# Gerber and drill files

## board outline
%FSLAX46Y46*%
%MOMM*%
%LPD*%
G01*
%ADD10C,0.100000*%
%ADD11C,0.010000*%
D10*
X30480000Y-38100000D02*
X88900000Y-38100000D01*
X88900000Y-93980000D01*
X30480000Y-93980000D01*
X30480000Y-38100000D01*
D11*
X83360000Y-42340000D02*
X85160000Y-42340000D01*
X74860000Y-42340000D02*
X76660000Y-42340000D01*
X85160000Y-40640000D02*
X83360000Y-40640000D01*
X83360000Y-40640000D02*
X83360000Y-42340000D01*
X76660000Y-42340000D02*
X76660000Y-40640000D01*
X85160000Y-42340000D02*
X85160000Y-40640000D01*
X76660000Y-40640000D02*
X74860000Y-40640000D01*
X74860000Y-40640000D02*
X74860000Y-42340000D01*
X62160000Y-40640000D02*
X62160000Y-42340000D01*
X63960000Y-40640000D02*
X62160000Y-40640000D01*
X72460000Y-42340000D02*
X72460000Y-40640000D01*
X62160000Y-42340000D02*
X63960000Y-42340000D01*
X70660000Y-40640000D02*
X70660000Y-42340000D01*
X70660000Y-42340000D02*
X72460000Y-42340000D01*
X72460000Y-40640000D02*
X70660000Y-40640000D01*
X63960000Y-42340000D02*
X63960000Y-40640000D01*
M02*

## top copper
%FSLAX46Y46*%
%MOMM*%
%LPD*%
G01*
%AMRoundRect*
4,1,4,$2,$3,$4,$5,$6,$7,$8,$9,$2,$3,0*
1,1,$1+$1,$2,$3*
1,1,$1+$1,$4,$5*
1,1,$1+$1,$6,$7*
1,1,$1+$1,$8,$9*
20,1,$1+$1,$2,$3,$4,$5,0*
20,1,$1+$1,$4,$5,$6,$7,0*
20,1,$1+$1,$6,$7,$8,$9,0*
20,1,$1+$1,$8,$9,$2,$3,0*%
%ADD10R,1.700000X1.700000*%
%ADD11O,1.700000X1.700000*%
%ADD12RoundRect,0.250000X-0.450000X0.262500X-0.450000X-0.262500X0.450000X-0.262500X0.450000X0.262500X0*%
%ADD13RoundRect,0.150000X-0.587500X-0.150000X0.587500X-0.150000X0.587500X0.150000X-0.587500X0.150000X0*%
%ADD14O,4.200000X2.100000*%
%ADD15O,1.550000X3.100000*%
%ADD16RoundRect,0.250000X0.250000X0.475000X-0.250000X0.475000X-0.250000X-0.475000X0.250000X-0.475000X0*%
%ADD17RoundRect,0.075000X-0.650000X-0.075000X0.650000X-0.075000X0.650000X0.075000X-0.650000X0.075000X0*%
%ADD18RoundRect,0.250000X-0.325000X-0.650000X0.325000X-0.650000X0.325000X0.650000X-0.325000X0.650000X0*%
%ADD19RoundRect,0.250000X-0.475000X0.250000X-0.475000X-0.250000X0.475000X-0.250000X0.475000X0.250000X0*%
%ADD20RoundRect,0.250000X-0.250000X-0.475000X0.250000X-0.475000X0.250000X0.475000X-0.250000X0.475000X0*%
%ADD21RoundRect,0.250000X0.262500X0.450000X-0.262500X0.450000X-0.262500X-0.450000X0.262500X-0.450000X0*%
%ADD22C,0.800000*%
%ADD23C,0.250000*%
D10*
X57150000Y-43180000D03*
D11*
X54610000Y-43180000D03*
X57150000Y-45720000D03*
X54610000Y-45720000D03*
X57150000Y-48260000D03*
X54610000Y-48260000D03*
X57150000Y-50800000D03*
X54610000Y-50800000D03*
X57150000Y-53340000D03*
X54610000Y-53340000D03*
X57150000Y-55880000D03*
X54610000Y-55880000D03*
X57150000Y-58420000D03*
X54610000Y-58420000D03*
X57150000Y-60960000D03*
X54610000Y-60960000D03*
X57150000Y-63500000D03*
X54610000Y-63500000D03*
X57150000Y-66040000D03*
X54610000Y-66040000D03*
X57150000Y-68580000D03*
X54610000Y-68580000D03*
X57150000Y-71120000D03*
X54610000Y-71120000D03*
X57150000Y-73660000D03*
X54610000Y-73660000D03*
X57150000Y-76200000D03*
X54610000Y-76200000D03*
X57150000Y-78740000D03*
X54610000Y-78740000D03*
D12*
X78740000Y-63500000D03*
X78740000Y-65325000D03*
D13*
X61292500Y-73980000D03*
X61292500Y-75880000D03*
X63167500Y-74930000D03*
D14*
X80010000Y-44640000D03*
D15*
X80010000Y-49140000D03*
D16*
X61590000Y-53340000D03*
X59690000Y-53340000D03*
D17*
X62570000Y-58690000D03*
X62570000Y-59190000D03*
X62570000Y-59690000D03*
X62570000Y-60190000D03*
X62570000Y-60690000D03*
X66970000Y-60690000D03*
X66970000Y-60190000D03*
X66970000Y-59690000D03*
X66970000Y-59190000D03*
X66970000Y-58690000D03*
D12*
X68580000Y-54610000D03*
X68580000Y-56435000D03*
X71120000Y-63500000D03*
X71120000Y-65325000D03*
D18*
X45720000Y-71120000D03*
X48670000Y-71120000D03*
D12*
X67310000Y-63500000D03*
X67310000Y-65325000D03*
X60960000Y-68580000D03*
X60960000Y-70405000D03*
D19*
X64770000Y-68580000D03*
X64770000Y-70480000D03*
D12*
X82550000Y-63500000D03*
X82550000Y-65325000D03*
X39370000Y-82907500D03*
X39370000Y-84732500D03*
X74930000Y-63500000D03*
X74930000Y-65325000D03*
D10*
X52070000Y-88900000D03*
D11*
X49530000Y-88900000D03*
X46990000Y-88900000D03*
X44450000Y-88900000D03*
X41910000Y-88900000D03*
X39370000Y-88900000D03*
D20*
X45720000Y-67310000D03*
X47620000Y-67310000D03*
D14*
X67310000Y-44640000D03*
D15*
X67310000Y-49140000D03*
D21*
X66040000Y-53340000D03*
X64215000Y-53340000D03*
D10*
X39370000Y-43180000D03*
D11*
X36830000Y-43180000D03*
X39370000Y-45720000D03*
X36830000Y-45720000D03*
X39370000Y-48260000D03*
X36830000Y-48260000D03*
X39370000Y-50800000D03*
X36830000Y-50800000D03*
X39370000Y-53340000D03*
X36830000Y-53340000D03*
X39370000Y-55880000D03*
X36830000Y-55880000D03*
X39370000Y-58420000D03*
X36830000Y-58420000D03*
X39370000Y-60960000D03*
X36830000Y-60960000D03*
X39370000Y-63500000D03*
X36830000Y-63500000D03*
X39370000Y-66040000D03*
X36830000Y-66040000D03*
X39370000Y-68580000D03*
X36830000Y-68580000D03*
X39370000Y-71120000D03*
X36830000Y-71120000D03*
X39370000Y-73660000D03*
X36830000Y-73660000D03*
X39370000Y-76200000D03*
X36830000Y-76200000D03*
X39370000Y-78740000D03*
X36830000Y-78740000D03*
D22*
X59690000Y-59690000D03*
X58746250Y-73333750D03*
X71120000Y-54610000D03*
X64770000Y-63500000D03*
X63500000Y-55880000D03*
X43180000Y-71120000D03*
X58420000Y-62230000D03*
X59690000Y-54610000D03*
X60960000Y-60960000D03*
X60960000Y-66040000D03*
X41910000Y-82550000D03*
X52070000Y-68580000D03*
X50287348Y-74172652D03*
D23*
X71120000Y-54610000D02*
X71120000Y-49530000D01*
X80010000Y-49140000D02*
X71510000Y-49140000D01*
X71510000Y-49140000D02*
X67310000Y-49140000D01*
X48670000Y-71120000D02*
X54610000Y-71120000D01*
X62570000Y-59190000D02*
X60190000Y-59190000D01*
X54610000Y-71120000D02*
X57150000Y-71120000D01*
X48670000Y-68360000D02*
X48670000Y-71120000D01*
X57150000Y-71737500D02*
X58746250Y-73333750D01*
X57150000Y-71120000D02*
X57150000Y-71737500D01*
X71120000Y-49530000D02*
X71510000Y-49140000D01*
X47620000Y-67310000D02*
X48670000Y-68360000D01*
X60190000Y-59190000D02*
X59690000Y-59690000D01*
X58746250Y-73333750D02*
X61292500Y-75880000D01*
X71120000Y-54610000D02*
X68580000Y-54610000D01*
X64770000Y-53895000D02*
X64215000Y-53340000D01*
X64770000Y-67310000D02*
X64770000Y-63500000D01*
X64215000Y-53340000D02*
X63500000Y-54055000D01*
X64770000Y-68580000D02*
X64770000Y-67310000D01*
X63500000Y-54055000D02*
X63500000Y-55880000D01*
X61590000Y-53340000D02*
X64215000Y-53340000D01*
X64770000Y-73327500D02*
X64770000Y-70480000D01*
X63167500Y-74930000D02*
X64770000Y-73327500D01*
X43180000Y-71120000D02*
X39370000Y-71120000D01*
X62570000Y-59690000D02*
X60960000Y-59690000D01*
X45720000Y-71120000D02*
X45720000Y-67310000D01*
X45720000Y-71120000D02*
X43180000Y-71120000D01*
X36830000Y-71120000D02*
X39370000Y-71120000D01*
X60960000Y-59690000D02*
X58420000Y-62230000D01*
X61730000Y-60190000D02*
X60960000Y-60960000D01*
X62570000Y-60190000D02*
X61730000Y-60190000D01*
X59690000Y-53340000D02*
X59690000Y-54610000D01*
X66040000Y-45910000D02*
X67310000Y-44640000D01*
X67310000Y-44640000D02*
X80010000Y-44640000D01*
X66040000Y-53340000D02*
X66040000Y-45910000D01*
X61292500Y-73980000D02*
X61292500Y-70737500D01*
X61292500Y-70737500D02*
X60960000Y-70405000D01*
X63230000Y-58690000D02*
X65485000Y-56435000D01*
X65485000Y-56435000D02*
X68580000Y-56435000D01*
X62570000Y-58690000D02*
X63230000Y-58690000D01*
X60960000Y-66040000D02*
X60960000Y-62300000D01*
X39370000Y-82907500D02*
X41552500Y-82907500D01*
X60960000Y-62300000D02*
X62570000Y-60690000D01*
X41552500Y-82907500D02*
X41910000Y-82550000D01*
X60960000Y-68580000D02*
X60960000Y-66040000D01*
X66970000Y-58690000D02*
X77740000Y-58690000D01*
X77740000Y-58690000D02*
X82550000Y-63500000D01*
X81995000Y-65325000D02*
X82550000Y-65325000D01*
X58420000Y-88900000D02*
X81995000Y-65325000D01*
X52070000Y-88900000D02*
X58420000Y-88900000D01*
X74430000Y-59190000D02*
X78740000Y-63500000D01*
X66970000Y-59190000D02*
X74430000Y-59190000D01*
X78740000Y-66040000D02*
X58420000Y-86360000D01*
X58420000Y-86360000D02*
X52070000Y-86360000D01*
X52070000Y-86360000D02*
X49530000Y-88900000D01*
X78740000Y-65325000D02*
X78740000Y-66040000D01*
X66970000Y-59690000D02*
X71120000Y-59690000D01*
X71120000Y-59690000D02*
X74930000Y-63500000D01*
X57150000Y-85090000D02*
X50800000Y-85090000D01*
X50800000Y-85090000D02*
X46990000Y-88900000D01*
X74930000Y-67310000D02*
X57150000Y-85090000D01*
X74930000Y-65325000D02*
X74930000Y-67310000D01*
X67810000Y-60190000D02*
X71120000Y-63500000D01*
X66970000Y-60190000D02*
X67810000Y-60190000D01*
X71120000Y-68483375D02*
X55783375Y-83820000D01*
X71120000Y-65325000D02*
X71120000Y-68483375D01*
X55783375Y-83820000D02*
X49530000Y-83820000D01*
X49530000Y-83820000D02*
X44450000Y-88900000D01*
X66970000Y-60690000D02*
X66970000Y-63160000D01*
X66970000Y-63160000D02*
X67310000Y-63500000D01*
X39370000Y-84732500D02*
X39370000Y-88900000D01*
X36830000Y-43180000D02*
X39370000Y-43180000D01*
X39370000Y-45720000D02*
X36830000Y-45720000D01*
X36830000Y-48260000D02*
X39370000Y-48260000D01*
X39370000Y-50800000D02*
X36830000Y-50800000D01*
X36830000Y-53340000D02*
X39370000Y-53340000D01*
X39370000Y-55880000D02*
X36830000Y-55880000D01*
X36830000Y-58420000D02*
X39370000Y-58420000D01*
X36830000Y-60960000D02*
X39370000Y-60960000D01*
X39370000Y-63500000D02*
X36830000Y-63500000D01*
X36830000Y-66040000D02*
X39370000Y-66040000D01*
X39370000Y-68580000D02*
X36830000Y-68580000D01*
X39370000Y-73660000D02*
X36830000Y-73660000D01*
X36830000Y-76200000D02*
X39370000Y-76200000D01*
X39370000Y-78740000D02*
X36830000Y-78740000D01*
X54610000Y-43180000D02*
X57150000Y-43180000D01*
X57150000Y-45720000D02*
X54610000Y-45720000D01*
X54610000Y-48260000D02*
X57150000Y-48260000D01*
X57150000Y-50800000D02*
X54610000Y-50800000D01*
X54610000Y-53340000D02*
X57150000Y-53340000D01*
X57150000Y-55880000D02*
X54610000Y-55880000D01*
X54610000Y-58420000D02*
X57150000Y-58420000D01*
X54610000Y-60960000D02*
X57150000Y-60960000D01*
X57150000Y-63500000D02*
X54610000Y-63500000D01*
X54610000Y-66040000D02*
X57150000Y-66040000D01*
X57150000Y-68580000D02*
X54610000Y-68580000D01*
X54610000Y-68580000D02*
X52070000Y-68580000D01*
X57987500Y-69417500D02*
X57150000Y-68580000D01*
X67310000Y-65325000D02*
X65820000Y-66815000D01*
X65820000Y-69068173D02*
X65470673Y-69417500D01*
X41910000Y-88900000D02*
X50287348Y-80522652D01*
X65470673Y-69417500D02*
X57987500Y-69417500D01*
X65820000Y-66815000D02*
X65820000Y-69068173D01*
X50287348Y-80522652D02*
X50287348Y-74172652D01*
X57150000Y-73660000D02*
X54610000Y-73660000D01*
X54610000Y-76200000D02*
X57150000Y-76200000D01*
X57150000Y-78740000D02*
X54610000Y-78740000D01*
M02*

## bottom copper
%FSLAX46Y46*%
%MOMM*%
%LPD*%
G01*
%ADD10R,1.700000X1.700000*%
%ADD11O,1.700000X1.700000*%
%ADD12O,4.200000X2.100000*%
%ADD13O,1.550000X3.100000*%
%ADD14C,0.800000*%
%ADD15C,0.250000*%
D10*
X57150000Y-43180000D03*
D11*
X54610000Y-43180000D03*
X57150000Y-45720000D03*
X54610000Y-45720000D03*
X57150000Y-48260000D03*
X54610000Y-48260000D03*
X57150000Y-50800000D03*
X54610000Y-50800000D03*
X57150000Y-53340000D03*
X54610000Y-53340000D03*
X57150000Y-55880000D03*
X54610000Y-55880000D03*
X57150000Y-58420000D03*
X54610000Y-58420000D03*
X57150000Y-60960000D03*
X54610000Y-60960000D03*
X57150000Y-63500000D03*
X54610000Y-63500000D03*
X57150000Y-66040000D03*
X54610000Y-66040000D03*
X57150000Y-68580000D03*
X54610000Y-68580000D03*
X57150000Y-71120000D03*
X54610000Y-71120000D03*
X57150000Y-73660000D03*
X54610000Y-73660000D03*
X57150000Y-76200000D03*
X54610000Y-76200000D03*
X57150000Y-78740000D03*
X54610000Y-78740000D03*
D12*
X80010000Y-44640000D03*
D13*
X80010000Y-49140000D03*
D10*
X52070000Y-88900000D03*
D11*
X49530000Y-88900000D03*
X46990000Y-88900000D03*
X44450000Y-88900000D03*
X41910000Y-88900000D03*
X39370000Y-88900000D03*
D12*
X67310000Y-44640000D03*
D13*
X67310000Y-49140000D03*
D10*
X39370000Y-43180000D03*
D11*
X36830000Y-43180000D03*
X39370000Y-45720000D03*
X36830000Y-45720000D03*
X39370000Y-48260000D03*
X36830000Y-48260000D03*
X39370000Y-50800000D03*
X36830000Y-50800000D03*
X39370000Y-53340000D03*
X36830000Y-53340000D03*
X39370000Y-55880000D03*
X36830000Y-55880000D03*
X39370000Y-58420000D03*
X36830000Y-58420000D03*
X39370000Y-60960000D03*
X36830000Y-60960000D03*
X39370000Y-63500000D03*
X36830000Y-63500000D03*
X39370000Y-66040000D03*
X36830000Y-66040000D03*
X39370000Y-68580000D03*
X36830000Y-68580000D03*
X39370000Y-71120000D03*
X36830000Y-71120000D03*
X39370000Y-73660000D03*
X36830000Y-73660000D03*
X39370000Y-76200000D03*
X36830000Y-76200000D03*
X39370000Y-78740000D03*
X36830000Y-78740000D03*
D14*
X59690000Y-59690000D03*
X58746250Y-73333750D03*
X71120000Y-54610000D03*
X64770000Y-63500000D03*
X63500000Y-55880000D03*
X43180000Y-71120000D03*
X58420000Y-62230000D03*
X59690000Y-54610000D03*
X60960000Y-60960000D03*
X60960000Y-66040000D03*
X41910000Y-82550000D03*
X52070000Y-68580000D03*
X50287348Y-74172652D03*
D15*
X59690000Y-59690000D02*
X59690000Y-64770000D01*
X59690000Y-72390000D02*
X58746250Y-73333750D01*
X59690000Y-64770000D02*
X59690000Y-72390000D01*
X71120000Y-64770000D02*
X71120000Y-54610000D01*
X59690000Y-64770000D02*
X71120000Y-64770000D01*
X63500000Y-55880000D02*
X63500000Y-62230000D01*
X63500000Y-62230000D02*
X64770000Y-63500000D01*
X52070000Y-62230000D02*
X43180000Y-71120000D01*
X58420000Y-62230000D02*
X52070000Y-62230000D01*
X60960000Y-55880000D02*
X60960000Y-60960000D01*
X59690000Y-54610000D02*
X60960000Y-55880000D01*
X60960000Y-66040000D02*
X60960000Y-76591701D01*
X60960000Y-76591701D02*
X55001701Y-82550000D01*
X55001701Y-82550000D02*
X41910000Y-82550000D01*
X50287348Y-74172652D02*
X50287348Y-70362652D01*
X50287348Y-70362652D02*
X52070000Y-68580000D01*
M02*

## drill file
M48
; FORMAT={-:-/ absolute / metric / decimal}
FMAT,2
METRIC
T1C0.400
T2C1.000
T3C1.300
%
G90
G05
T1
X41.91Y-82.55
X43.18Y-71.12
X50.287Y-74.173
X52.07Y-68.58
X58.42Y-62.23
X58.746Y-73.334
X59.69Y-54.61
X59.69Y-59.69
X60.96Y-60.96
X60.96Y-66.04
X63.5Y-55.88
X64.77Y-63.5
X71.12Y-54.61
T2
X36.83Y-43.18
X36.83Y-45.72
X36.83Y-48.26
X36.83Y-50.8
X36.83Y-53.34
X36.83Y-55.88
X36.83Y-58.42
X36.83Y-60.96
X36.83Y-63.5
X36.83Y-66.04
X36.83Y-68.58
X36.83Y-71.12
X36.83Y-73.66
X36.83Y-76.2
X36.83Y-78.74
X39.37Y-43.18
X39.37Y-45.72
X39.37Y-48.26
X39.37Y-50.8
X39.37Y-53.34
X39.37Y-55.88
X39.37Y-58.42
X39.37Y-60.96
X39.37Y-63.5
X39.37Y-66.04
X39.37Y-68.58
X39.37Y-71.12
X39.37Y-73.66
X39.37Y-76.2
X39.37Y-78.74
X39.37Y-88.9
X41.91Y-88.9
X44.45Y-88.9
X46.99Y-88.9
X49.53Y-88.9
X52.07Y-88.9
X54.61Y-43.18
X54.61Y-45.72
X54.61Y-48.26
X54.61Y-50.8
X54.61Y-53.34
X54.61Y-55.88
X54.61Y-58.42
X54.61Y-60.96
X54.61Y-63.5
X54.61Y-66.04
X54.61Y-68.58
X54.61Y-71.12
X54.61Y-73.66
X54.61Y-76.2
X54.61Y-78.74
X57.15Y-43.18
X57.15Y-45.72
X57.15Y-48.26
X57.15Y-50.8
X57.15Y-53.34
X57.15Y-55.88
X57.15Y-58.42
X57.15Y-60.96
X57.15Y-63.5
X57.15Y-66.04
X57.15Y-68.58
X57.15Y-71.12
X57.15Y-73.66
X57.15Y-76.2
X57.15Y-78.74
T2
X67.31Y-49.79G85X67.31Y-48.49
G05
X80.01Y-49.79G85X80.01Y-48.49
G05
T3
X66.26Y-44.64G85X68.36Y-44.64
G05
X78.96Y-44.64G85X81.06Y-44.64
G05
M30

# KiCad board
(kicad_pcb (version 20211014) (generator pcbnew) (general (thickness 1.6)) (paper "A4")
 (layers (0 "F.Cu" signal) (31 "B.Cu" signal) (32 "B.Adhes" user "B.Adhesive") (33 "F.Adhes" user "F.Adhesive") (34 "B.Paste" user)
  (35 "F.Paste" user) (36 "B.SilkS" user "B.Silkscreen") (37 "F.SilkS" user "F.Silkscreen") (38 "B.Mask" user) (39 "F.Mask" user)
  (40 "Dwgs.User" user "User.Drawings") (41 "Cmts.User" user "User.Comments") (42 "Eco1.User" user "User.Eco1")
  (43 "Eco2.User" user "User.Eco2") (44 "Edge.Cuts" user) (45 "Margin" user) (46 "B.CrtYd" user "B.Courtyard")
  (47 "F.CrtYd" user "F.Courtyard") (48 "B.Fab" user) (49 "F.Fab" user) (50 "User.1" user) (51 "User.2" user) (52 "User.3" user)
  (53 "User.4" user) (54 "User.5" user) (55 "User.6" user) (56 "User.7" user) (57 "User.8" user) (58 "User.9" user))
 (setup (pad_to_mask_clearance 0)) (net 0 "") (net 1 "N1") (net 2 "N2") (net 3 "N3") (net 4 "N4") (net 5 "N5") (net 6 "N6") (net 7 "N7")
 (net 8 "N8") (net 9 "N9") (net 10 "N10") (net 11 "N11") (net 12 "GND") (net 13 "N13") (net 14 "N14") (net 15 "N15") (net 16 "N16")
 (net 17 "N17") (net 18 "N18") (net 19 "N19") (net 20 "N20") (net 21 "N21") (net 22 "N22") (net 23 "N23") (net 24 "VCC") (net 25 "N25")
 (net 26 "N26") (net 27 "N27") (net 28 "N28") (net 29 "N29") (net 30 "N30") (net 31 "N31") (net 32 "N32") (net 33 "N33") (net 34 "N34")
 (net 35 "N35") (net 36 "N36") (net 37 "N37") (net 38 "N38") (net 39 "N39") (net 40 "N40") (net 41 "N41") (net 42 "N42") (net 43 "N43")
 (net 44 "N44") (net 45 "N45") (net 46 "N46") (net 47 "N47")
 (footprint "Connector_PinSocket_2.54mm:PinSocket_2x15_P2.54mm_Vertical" (layer "F.Cu") (at 57.15 43.18)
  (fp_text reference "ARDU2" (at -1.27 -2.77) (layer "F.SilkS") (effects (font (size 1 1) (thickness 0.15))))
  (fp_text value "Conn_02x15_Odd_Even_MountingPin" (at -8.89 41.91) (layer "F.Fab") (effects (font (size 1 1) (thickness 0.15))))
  (pad "1" thru_hole rect (at 0 0) (size 1.7 1.7) (drill 1) (layers *.Cu *.Mask) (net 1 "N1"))
  (pad "2" thru_hole oval (at -2.54 0) (size 1.7 1.7) (drill 1) (layers *.Cu *.Mask) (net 1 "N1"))
  (pad "3" thru_hole oval (at 0 2.54) (size 1.7 1.7) (drill 1) (layers *.Cu *.Mask) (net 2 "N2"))
  (pad "4" thru_hole oval (at -2.54 2.54) (size 1.7 1.7) (drill 1) (layers *.Cu *.Mask) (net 2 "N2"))
  (pad "5" thru_hole oval (at 0 5.08) (size 1.7 1.7) (drill 1) (layers *.Cu *.Mask) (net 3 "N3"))
  (pad "6" thru_hole oval (at -2.54 5.08) (size 1.7 1.7) (drill 1) (layers *.Cu *.Mask) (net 3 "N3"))
  (pad "7" thru_hole oval (at 0 7.62) (size 1.7 1.7) (drill 1) (layers *.Cu *.Mask) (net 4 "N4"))
  (pad "8" thru_hole oval (at -2.54 7.62) (size 1.7 1.7) (drill 1) (layers *.Cu *.Mask) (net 4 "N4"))
  (pad "9" thru_hole oval (at 0 10.16) (size 1.7 1.7) (drill 1) (layers *.Cu *.Mask) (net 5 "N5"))
  (pad "10" thru_hole oval (at -2.54 10.16) (size 1.7 1.7) (drill 1) (layers *.Cu *.Mask) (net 5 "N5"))
  (pad "11" thru_hole oval (at 0 12.7) (size 1.7 1.7) (drill 1) (layers *.Cu *.Mask) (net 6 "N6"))
  (pad "12" thru_hole oval (at -2.54 12.7) (size 1.7 1.7) (drill 1) (layers *.Cu *.Mask) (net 6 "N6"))
  (pad "13" thru_hole oval (at 0 15.24) (size 1.7 1.7) (drill 1) (layers *.Cu *.Mask) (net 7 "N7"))
  (pad "14" thru_hole oval (at -2.54 15.24) (size 1.7 1.7) (drill 1) (layers *.Cu *.Mask) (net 7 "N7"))
  (pad "15" thru_hole oval (at 0 17.78) (size 1.7 1.7) (drill 1) (layers *.Cu *.Mask) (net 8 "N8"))
  (pad "16" thru_hole oval (at -2.54 17.78) (size 1.7 1.7) (drill 1) (layers *.Cu *.Mask) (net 8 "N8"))
  (pad "17" thru_hole oval (at 0 20.32) (size 1.7 1.7) (drill 1) (layers *.Cu *.Mask) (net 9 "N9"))
  (pad "18" thru_hole oval (at -2.54 20.32) (size 1.7 1.7) (drill 1) (layers *.Cu *.Mask) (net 9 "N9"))
  (pad "19" thru_hole oval (at 0 22.86) (size 1.7 1.7) (drill 1) (layers *.Cu *.Mask) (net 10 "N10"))
  (pad "20" thru_hole oval (at -2.54 22.86) (size 1.7 1.7) (drill 1) (layers *.Cu *.Mask) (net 10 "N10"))
  (pad "21" thru_hole oval (at 0 25.4) (size 1.7 1.7) (drill 1) (layers *.Cu *.Mask) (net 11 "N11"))
  (pad "22" thru_hole oval (at -2.54 25.4) (size 1.7 1.7) (drill 1) (layers *.Cu *.Mask) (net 11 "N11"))
  (pad "23" thru_hole oval (at 0 27.94) (size 1.7 1.7) (drill 1) (layers *.Cu *.Mask) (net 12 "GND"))
  (pad "24" thru_hole oval (at -2.54 27.94) (size 1.7 1.7) (drill 1) (layers *.Cu *.Mask) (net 12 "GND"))
  (pad "25" thru_hole oval (at 0 30.48) (size 1.7 1.7) (drill 1) (layers *.Cu *.Mask) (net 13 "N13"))
  (pad "26" thru_hole oval (at -2.54 30.48) (size 1.7 1.7) (drill 1) (layers *.Cu *.Mask) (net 13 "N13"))
  (pad "27" thru_hole oval (at 0 33.02) (size 1.7 1.7) (drill 1) (layers *.Cu *.Mask) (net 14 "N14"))
  (pad "28" thru_hole oval (at -2.54 33.02) (size 1.7 1.7) (drill 1) (layers *.Cu *.Mask) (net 14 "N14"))
  (pad "29" thru_hole oval (at 0 35.56) (size 1.7 1.7) (drill 1) (layers *.Cu *.Mask) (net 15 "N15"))
  (pad "30" thru_hole oval (at -2.54 35.56) (size 1.7 1.7) (drill 1) (layers *.Cu *.Mask) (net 15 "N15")))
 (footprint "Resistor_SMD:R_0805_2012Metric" (layer "F.Cu") (at 78.74 64.4125 -90)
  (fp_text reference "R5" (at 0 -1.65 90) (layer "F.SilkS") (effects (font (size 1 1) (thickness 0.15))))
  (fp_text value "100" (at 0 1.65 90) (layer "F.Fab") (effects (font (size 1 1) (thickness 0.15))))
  (pad "1" smd roundrect (at -0.9125 0 270) (size 1.025 1.4) (layers "F.Cu" "F.Paste" "F.Mask") (roundrect_rratio 0.243902) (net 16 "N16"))
  (pad "2" smd roundrect (at 0.9125 0 270) (size 1.025 1.4) (layers "F.Cu" "F.Paste" "F.Mask") (roundrect_rratio 0.243902) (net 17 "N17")))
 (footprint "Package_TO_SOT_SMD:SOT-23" (layer "F.Cu") (at 62.23 74.93)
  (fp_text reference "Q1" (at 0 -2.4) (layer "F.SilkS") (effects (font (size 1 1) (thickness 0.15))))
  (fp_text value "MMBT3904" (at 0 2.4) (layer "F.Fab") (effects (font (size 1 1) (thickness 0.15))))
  (pad "1" smd roundrect (at -0.9375 -0.95) (size 1.475 0.6) (layers "F.Cu" "F.Paste" "F.Mask") (roundrect_rratio 0.25) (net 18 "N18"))
  (pad "2" smd roundrect (at -0.9375 0.95) (size 1.475 0.6) (layers "F.Cu" "F.Paste" "F.Mask") (roundrect_rratio 0.25) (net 12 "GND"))
  (pad "3" smd roundrect (at 0.9375 0) (size 1.475 0.6) (layers "F.Cu" "F.Paste" "F.Mask") (roundrect_rratio 0.25) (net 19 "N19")))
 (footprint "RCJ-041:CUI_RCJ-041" (layer "F.Cu") (at 80.01 40.64 90)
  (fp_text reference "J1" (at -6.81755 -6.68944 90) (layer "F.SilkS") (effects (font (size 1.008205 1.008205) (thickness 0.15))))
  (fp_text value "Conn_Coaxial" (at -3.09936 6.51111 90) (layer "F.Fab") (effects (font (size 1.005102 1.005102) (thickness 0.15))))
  (fp_line (start -1.7 3.35) (end -1.7 5.15) (layer "Edge.Cuts") (width 0.01))
  (fp_line (start -1.7 -5.15) (end -1.7 -3.35) (layer "Edge.Cuts") (width 0.01))
  (fp_line (start 0 5.15) (end 0 3.35) (layer "Edge.Cuts") (width 0.01))
  (fp_line (start 0 3.35) (end -1.7 3.35) (layer "Edge.Cuts") (width 0.01))
  (fp_line (start -1.7 -3.35) (end 0 -3.35) (layer "Edge.Cuts") (width 0.01))
  (fp_line (start -1.7 5.15) (end 0 5.15) (layer "Edge.Cuts") (width 0.01))
  (fp_line (start 0 -3.35) (end 0 -5.15) (layer "Edge.Cuts") (width 0.01))
  (fp_line (start 0 -5.15) (end -1.7 -5.15) (layer "Edge.Cuts") (width 0.01))
  (pad "1" thru_hole oval locked (at -4 0 90) (size 2.1 4.2) (drill oval 1.3 3.4) (layers *.Cu *.Mask) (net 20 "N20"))
  (pad "2" thru_hole oval locked (at -8.5 0 90) (size 3.1 1.55) (drill oval 2.3 1) (layers *.Cu *.Mask) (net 12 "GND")))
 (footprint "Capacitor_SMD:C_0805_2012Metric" (layer "F.Cu") (at 60.64 53.34 180)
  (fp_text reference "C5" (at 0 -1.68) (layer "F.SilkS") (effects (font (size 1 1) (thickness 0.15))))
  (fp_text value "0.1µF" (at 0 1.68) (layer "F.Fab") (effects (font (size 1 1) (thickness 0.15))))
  (pad "1" smd roundrect (at -0.95 0 180) (size 1 1.45) (layers "F.Cu" "F.Paste" "F.Mask") (roundrect_rratio 0.25) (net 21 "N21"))
  (pad "2" smd roundrect (at 0.95 0 180) (size 1 1.45) (layers "F.Cu" "F.Paste" "F.Mask") (roundrect_rratio 0.25) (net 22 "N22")))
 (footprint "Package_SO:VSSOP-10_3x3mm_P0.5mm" (layer "F.Cu") (at 64.77 59.69)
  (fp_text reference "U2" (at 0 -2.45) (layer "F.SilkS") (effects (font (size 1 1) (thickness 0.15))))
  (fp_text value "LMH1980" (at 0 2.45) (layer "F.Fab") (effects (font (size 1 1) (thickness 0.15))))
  (pad "1" smd roundrect (at -2.2 -1) (size 1.45 0.3) (layers "F.Cu" "F.Paste" "F.Mask") (roundrect_rratio 0.25) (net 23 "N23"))
  (pad "2" smd roundrect (at -2.2 -0.5) (size 1.45 0.3) (layers "F.Cu" "F.Paste" "F.Mask") (roundrect_rratio 0.25) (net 12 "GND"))
  (pad "3" smd roundrect (at -2.2 0) (size 1.45 0.3) (layers "F.Cu" "F.Paste" "F.Mask") (roundrect_rratio 0.25) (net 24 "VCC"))
  (pad "4" smd roundrect (at -2.2 0.5) (size 1.45 0.3) (layers "F.Cu" "F.Paste" "F.Mask") (roundrect_rratio 0.25) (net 22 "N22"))
  (pad "5" smd roundrect (at -2.2 1) (size 1.45 0.3) (layers "F.Cu" "F.Paste" "F.Mask") (roundrect_rratio 0.25) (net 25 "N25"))
  (pad "6" smd roundrect (at 2.2 1) (size 1.45 0.3) (layers "F.Cu" "F.Paste" "F.Mask") (roundrect_rratio 0.25) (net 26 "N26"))
  (pad "7" smd roundrect (at 2.2 0.5) (size 1.45 0.3) (layers "F.Cu" "F.Paste" "F.Mask") (roundrect_rratio 0.25) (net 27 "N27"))
  (pad "8" smd roundrect (at 2.2 0) (size 1.45 0.3) (layers "F.Cu" "F.Paste" "F.Mask") (roundrect_rratio 0.25) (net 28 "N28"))
  (pad "9" smd roundrect (at 2.2 -0.5) (size 1.45 0.3) (layers "F.Cu" "F.Paste" "F.Mask") (roundrect_rratio 0.25) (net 16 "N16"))
  (pad "10" smd roundrect (at 2.2 -1) (size 1.45 0.3) (layers "F.Cu" "F.Paste" "F.Mask") (roundrect_rratio 0.25) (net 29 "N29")))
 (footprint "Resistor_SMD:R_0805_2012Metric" (layer "F.Cu") (at 68.58 55.5225 -90)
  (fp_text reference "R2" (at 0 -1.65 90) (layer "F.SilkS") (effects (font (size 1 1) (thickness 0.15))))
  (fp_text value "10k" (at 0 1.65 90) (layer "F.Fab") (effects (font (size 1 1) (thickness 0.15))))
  (pad "1" smd roundrect (at -0.9125 0 270) (size 1.025 1.4) (layers "F.Cu" "F.Paste" "F.Mask") (roundrect_rratio 0.243902) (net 12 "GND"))
  (pad "2" smd roundrect (at 0.9125 0 270) (size 1.025 1.4) (layers "F.Cu" "F.Paste" "F.Mask") (roundrect_rratio 0.243902) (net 23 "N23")))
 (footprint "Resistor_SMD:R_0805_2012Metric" (layer "F.Cu") (at 71.12 64.4125 -90)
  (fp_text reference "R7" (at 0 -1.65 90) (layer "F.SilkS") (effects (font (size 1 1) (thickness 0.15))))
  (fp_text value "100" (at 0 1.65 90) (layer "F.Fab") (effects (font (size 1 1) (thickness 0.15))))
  (pad "1" smd roundrect (at -0.9125 0 270) (size 1.025 1.4) (layers "F.Cu" "F.Paste" "F.Mask") (roundrect_rratio 0.243902) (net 27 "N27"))
  (pad "2" smd roundrect (at 0.9125 0 270) (size 1.025 1.4) (layers "F.Cu" "F.Paste" "F.Mask") (roundrect_rratio 0.243902) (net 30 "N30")))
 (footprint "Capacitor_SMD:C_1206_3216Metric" (layer "F.Cu") (at 47.195 71.12)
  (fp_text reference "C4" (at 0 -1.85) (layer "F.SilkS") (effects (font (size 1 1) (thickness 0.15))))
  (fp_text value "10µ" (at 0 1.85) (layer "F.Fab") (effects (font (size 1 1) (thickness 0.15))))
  (pad "1" smd roundrect (at -1.475 0) (size 1.15 1.8) (layers "F.Cu" "F.Paste" "F.Mask") (roundrect_rratio 0.217391) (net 24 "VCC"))
  (pad "2" smd roundrect (at 1.475 0) (size 1.15 1.8) (layers "F.Cu" "F.Paste" "F.Mask") (roundrect_rratio 0.217391) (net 12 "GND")))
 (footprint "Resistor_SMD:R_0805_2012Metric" (layer "F.Cu") (at 67.31 64.4125 -90)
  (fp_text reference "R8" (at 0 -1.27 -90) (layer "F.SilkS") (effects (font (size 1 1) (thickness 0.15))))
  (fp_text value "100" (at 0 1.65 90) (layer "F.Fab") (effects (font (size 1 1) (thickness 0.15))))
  (pad "1" smd roundrect (at -0.9125 0 270) (size 1.025 1.4) (layers "F.Cu" "F.Paste" "F.Mask") (roundrect_rratio 0.243902) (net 26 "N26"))
  (pad "2" smd roundrect (at 0.9125 0 270) (size 1.025 1.4) (layers "F.Cu" "F.Paste" "F.Mask") (roundrect_rratio 0.243902) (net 11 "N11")))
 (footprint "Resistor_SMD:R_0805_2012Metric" (layer "F.Cu") (at 60.96 69.4925 -90)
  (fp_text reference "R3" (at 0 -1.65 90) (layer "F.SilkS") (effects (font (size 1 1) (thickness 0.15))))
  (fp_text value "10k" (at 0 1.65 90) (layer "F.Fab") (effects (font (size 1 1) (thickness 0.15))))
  (pad "1" smd roundrect (at -0.9125 0 270) (size 1.025 1.4) (layers "F.Cu" "F.Paste" "F.Mask") (roundrect_rratio 0.243902) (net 25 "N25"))
  (pad "2" smd roundrect (at 0.9125 0 270) (size 1.025 1.4) (layers "F.Cu" "F.Paste" "F.Mask") (roundrect_rratio 0.243902) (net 18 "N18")))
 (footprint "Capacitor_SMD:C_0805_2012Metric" (layer "F.Cu") (at 64.77 69.53 -90)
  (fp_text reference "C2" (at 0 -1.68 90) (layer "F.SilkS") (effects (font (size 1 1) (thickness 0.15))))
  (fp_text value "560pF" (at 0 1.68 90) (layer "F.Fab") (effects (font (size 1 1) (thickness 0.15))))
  (pad "1" smd roundrect (at -0.95 0 270) (size 1 1.45) (layers "F.Cu" "F.Paste" "F.Mask") (roundrect_rratio 0.25) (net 21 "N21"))
  (pad "2" smd roundrect (at 0.95 0 270) (size 1 1.45) (layers "F.Cu" "F.Paste" "F.Mask") (roundrect_rratio 0.25) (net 19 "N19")))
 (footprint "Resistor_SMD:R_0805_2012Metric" (layer "F.Cu") (at 82.55 64.4125 -90)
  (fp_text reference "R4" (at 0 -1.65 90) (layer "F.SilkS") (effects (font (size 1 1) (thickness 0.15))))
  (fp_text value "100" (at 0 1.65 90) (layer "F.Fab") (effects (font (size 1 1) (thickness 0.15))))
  (pad "1" smd roundrect (at -0.9125 0 270) (size 1.025 1.4) (layers "F.Cu" "F.Paste" "F.Mask") (roundrect_rratio 0.243902) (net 29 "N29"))
  (pad "2" smd roundrect (at 0.9125 0 270) (size 1.025 1.4) (layers "F.Cu" "F.Paste" "F.Mask") (roundrect_rratio 0.243902) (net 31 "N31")))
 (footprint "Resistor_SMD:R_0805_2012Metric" (layer "F.Cu") (at 39.37 83.82 -90)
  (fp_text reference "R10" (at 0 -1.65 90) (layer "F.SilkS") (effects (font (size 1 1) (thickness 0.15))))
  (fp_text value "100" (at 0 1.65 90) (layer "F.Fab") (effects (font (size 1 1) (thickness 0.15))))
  (pad "1" smd roundrect (at -0.9125 0 270) (size 1.025 1.4) (layers "F.Cu" "F.Paste" "F.Mask") (roundrect_rratio 0.243902) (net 25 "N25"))
  (pad "2" smd roundrect (at 0.9125 0 270) (size 1.025 1.4) (layers "F.Cu" "F.Paste" "F.Mask") (roundrect_rratio 0.243902) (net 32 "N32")))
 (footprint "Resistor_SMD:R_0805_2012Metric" (layer "F.Cu") (at 74.93 64.4125 -90)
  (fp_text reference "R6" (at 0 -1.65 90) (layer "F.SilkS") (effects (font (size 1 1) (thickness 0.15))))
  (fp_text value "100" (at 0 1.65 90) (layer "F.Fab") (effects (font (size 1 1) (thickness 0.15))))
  (pad "1" smd roundrect (at -0.9125 0 270) (size 1.025 1.4) (layers "F.Cu" "F.Paste" "F.Mask") (roundrect_rratio 0.243902) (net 28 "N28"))
  (pad "2" smd roundrect (at 0.9125 0 270) (size 1.025 1.4) (layers "F.Cu" "F.Paste" "F.Mask") (roundrect_rratio 0.243902) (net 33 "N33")))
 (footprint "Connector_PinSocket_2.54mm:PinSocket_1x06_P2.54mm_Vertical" (layer "F.Cu") (at 52.07 88.9 -90)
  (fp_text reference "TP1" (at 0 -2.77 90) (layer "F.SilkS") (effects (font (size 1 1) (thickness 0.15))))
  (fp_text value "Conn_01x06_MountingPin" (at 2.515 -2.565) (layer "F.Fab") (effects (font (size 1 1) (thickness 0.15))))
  (pad "1" thru_hole rect (at 0 0 270) (size 1.7 1.7) (drill 1) (layers *.Cu *.Mask) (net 31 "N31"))
  (pad "2" thru_hole oval (at 0 2.54 270) (size 1.7 1.7) (drill 1) (layers *.Cu *.Mask) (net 17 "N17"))
  (pad "3" thru_hole oval (at 0 5.08 270) (size 1.7 1.7) (drill 1) (layers *.Cu *.Mask) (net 33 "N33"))
  (pad "4" thru_hole oval (at 0 7.62 270) (size 1.7 1.7) (drill 1) (layers *.Cu *.Mask) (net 30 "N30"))
  (pad "5" thru_hole oval (at 0 10.16 270) (size 1.7 1.7) (drill 1) (layers *.Cu *.Mask) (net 11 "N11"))
  (pad "6" thru_hole oval (at 0 12.7 270) (size 1.7 1.7) (drill 1) (layers *.Cu *.Mask) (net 32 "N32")))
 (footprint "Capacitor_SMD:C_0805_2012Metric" (layer "F.Cu") (at 46.67 67.31)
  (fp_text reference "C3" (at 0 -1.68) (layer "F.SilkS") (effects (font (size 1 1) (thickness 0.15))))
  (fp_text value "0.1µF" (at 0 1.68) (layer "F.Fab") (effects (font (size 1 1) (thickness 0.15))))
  (pad "1" smd roundrect (at -0.95 0) (size 1 1.45) (layers "F.Cu" "F.Paste" "F.Mask") (roundrect_rratio 0.25) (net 24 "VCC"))
  (pad "2" smd roundrect (at 0.95 0) (size 1 1.45) (layers "F.Cu" "F.Paste" "F.Mask") (roundrect_rratio 0.25) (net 12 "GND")))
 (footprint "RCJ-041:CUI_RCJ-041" (layer "F.Cu") (at 67.31 40.64 90)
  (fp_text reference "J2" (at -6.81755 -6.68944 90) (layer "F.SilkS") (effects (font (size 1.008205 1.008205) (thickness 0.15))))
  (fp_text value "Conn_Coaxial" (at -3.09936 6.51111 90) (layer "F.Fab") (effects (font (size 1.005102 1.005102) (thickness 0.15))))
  (fp_line (start 0 -5.15) (end -1.7 -5.15) (layer "Edge.Cuts") (width 0.01))
  (fp_line (start 0 -3.35) (end 0 -5.15) (layer "Edge.Cuts") (width 0.01))
  (fp_line (start -1.7 5.15) (end 0 5.15) (layer "Edge.Cuts") (width 0.01))
  (fp_line (start -1.7 -5.15) (end -1.7 -3.35) (layer "Edge.Cuts") (width 0.01))
  (fp_line (start 0 3.35) (end -1.7 3.35) (layer "Edge.Cuts") (width 0.01))
  (fp_line (start -1.7 3.35) (end -1.7 5.15) (layer "Edge.Cuts") (width 0.01))
  (fp_line (start 0 5.15) (end 0 3.35) (layer "Edge.Cuts") (width 0.01))
  (fp_line (start -1.7 -3.35) (end 0 -3.35) (layer "Edge.Cuts") (width 0.01))
  (pad "1" thru_hole oval locked (at -4 0 90) (size 2.1 4.2) (drill oval 1.3 3.4) (layers *.Cu *.Mask) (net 20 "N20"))
  (pad "2" thru_hole oval locked (at -8.5 0 90) (size 3.1 1.55) (drill oval 2.3 1) (layers *.Cu *.Mask) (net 12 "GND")))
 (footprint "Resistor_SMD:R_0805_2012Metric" (layer "F.Cu") (at 65.1275 53.34 180)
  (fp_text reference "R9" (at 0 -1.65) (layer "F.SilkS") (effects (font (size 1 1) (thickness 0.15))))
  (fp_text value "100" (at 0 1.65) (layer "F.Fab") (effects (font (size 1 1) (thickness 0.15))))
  (pad "1" smd roundrect (at -0.9125 0 180) (size 1.025 1.4) (layers "F.Cu" "F.Paste" "F.Mask") (roundrect_rratio 0.243902) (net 20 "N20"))
  (pad "2" smd roundrect (at 0.9125 0 180) (size 1.025 1.4) (layers "F.Cu" "F.Paste" "F.Mask") (roundrect_rratio 0.243902) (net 21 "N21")))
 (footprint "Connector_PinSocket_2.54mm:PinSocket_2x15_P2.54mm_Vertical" (layer "F.Cu") (at 39.37 43.18)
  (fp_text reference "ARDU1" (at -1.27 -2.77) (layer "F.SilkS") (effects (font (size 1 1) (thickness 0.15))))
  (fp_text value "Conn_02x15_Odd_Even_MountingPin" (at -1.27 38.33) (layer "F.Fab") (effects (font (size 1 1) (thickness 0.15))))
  (pad "1" thru_hole rect (at 0 0) (size 1.7 1.7) (drill 1) (layers *.Cu *.Mask) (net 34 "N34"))
  (pad "2" thru_hole oval (at -2.54 0) (size 1.7 1.7) (drill 1) (layers *.Cu *.Mask) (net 34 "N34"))
  (pad "3" thru_hole oval (at 0 2.54) (size 1.7 1.7) (drill 1) (layers *.Cu *.Mask) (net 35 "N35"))
  (pad "4" thru_hole oval (at -2.54 2.54) (size 1.7 1.7) (drill 1) (layers *.Cu *.Mask) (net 35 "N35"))
  (pad "5" thru_hole oval (at 0 5.08) (size 1.7 1.7) (drill 1) (layers *.Cu *.Mask) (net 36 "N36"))
  (pad "6" thru_hole oval (at -2.54 5.08) (size 1.7 1.7) (drill 1) (layers *.Cu *.Mask) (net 36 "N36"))
  (pad "7" thru_hole oval (at 0 7.62) (size 1.7 1.7) (drill 1) (layers *.Cu *.Mask) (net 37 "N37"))
  (pad "8" thru_hole oval (at -2.54 7.62) (size 1.7 1.7) (drill 1) (layers *.Cu *.Mask) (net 37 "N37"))
  (pad "9" thru_hole oval (at 0 10.16) (size 1.7 1.7) (drill 1) (layers *.Cu *.Mask) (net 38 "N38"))
  (pad "10" thru_hole oval (at -2.54 10.16) (size 1.7 1.7) (drill 1) (layers *.Cu *.Mask) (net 38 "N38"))
  (pad "11" thru_hole oval (at 0 12.7) (size 1.7 1.7) (drill 1) (layers *.Cu *.Mask) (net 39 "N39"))
  (pad "12" thru_hole oval (at -2.54 12.7) (size 1.7 1.7) (drill 1) (layers *.Cu *.Mask) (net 39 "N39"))
  (pad "13" thru_hole oval (at 0 15.24) (size 1.7 1.7) (drill 1) (layers *.Cu *.Mask) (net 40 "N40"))
  (pad "14" thru_hole oval (at -2.54 15.24) (size 1.7 1.7) (drill 1) (layers *.Cu *.Mask) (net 40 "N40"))
  (pad "15" thru_hole oval (at 0 17.78) (size 1.7 1.7) (drill 1) (layers *.Cu *.Mask) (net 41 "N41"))
  (pad "16" thru_hole oval (at -2.54 17.78) (size 1.7 1.7) (drill 1) (layers *.Cu *.Mask) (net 41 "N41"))
  (pad "17" thru_hole oval (at 0 20.32) (size 1.7 1.7) (drill 1) (layers *.Cu *.Mask) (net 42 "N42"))
  (pad "18" thru_hole oval (at -2.54 20.32) (size 1.7 1.7) (drill 1) (layers *.Cu *.Mask) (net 42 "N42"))
  (pad "19" thru_hole oval (at 0 22.86) (size 1.7 1.7) (drill 1) (layers *.Cu *.Mask) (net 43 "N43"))
  (pad "20" thru_hole oval (at -2.54 22.86) (size 1.7 1.7) (drill 1) (layers *.Cu *.Mask) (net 43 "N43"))
  (pad "21" thru_hole oval (at 0 25.4) (size 1.7 1.7) (drill 1) (layers *.Cu *.Mask) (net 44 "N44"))
  (pad "22" thru_hole oval (at -2.54 25.4) (size 1.7 1.7) (drill 1) (layers *.Cu *.Mask) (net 44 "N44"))
  (pad "23" thru_hole oval (at 0 27.94) (size 1.7 1.7) (drill 1) (layers *.Cu *.Mask) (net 24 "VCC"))
  (pad "24" thru_hole oval (at -2.54 27.94) (size 1.7 1.7) (drill 1) (layers *.Cu *.Mask) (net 24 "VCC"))
  (pad "25" thru_hole oval (at 0 30.48) (size 1.7 1.7) (drill 1) (layers *.Cu *.Mask) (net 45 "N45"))
  (pad "26" thru_hole oval (at -2.54 30.48) (size 1.7 1.7) (drill 1) (layers *.Cu *.Mask) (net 45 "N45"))
  (pad "27" thru_hole oval (at 0 33.02) (size 1.7 1.7) (drill 1) (layers *.Cu *.Mask) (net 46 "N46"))
  (pad "28" thru_hole oval (at -2.54 33.02) (size 1.7 1.7) (drill 1) (layers *.Cu *.Mask) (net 46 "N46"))
  (pad "29" thru_hole oval (at 0 35.56) (size 1.7 1.7) (drill 1) (layers *.Cu *.Mask) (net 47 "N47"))
  (pad "30" thru_hole oval (at -2.54 35.56) (size 1.7 1.7) (drill 1) (layers *.Cu *.Mask) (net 47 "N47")))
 (gr_rect (start 88.9 38.1) (end 30.48 93.98) (layer "Edge.Cuts") (width 0.1) (fill none))
 (segment (start 71.12 54.61) (end 71.12 49.53) (width 0.25) (layer "F.Cu") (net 12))
 (segment (start 80.01 49.14) (end 71.51 49.14) (width 0.25) (layer "F.Cu") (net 12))
 (segment (start 71.51 49.14) (end 67.31 49.14) (width 0.25) (layer "F.Cu") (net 12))
 (segment (start 48.67 71.12) (end 54.61 71.12) (width 0.25) (layer "F.Cu") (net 12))
 (segment (start 62.57 59.19) (end 60.19 59.19) (width 0.25) (layer "F.Cu") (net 12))
 (segment (start 54.61 71.12) (end 57.15 71.12) (width 0.25) (layer "F.Cu") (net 12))
 (segment (start 48.67 68.36) (end 48.67 71.12) (width 0.25) (layer "F.Cu") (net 12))
 (segment (start 57.15 71.7375) (end 58.74625 73.33375) (width 0.25) (layer "F.Cu") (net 12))
 (segment (start 57.15 71.12) (end 57.15 71.7375) (width 0.25) (layer "F.Cu") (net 12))
 (segment (start 71.12 49.53) (end 71.51 49.14) (width 0.25) (layer "F.Cu") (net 12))
 (segment (start 47.62 67.31) (end 48.67 68.36) (width 0.25) (layer "F.Cu") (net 12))
 (segment (start 60.19 59.19) (end 59.69 59.69) (width 0.25) (layer "F.Cu") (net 12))
 (segment (start 58.74625 73.33375) (end 61.2925 75.88) (width 0.25) (layer "F.Cu") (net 12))
 (segment (start 71.12 54.61) (end 68.58 54.61) (width 0.25) (layer "F.Cu") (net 12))
 (via (at 59.69 59.69) (size 0.8) (drill 0.4) (layers "F.Cu" "B.Cu") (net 12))
 (via (at 58.74625 73.33375) (size 0.8) (drill 0.4) (layers "F.Cu" "B.Cu") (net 12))
 (via (at 71.12 54.61) (size 0.8) (drill 0.4) (layers "F.Cu" "B.Cu") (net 12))
 (segment (start 59.69 59.69) (end 59.69 64.77) (width 0.25) (layer "B.Cu") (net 12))
 (segment (start 59.69 72.39) (end 58.74625 73.33375) (width 0.25) (layer "B.Cu") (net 12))
 (segment (start 59.69 64.77) (end 59.69 72.39) (width 0.25) (layer "B.Cu") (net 12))
 (segment (start 71.12 64.77) (end 71.12 54.61) (width 0.25) (layer "B.Cu") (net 12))
 (segment (start 59.69 64.77) (end 71.12 64.77) (width 0.25) (layer "B.Cu") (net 12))
 (segment (start 64.77 53.895) (end 64.215 53.34) (width 0.25) (layer "F.Cu") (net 21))
 (segment (start 64.77 67.31) (end 64.77 63.5) (width 0.25) (layer "F.Cu") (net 21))
 (segment (start 64.215 53.34) (end 63.5 54.055) (width 0.25) (layer "F.Cu") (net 21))
 (segment (start 64.77 68.58) (end 64.77 67.31) (width 0.25) (layer "F.Cu") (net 21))
 (segment (start 63.5 54.055) (end 63.5 55.88) (width 0.25) (layer "F.Cu") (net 21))
 (segment (start 61.59 53.34) (end 64.215 53.34) (width 0.25) (layer "F.Cu") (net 21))
 (via (at 64.77 63.5) (size 0.8) (drill 0.4) (layers "F.Cu" "B.Cu") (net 21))
 (via (at 63.5 55.88) (size 0.8) (drill 0.4) (layers "F.Cu" "B.Cu") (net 21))
 (segment (start 63.5 55.88) (end 63.5 62.23) (width 0.25) (layer "B.Cu") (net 21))
 (segment (start 63.5 62.23) (end 64.77 63.5) (width 0.25) (layer "B.Cu") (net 21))
 (segment (start 64.77 73.3275) (end 64.77 70.48) (width 0.25) (layer "F.Cu") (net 19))
 (segment (start 63.1675 74.93) (end 64.77 73.3275) (width 0.25) (layer "F.Cu") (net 19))
 (segment (start 43.18 71.12) (end 39.37 71.12) (width 0.25) (layer "F.Cu") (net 24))
 (segment (start 62.57 59.69) (end 60.96 59.69) (width 0.25) (layer "F.Cu") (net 24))
 (segment (start 45.72 71.12) (end 45.72 67.31) (width 0.25) (layer "F.Cu") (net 24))
 (segment (start 45.72 71.12) (end 43.18 71.12) (width 0.25) (layer "F.Cu") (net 24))
 (segment (start 36.83 71.12) (end 39.37 71.12) (width 0.25) (layer "F.Cu") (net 24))
 (segment (start 60.96 59.69) (end 58.42 62.23) (width 0.25) (layer "F.Cu") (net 24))
 (via (at 43.18 71.12) (size 0.8) (drill 0.4) (layers "F.Cu" "B.Cu") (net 24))
 (via (at 58.42 62.23) (size 0.8) (drill 0.4) (layers "F.Cu" "B.Cu") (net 24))
 (segment (start 52.07 62.23) (end 43.18 71.12) (width 0.25) (layer "B.Cu") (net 24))
 (segment (start 58.42 62.23) (end 52.07 62.23) (width 0.25) (layer "B.Cu") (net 24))
 (segment (start 61.73 60.19) (end 60.96 60.96) (width 0.25) (layer "F.Cu") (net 22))
 (segment (start 62.57 60.19) (end 61.73 60.19) (width 0.25) (layer "F.Cu") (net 22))
 (segment (start 59.69 53.34) (end 59.69 54.61) (width 0.25) (layer "F.Cu") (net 22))
 (via (at 59.69 54.61) (size 0.8) (drill 0.4) (layers "F.Cu" "B.Cu") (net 22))
 (via (at 60.96 60.96) (size 0.8) (drill 0.4) (layers "F.Cu" "B.Cu") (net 22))
 (segment (start 60.96 55.88) (end 60.96 60.96) (width 0.25) (layer "B.Cu") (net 22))
 (segment (start 59.69 54.61) (end 60.96 55.88) (width 0.25) (layer "B.Cu") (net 22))
 (segment (start 66.04 45.91) (end 67.31 44.64) (width 0.25) (layer "F.Cu") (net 20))
 (segment (start 67.31 44.64) (end 80.01 44.64) (width 0.25) (layer "F.Cu") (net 20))
 (segment (start 66.04 53.34) (end 66.04 45.91) (width 0.25) (layer "F.Cu") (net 20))
 (segment (start 61.2925 73.98) (end 61.2925 70.7375) (width 0.25) (layer "F.Cu") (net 18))
 (segment (start 61.2925 70.7375) (end 60.96 70.405) (width 0.25) (layer "F.Cu") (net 18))
 (segment (start 63.23 58.69) (end 65.485 56.435) (width 0.25) (layer "F.Cu") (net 23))
 (segment (start 65.485 56.435) (end 68.58 56.435) (width 0.25) (layer "F.Cu") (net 23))
 (segment (start 62.57 58.69) (end 63.23 58.69) (width 0.25) (layer "F.Cu") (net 23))
 (segment (start 60.96 66.04) (end 60.96 62.3) (width 0.25) (layer "F.Cu") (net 25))
 (segment (start 39.37 82.9075) (end 41.5525 82.9075) (width 0.25) (layer "F.Cu") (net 25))
 (segment (start 60.96 62.3) (end 62.57 60.69) (width 0.25) (layer "F.Cu") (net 25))
 (segment (start 41.5525 82.9075) (end 41.91 82.55) (width 0.25) (layer "F.Cu") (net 25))
 (segment (start 60.96 68.58) (end 60.96 66.04) (width 0.25) (layer "F.Cu") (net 25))
 (via (at 60.96 66.04) (size 0.8) (drill 0.4) (layers "F.Cu" "B.Cu") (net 25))
 (via (at 41.91 82.55) (size 0.8) (drill 0.4) (layers "F.Cu" "B.Cu") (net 25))
 (segment (start 60.96 66.04) (end 60.96 76.591701) (width 0.25) (layer "B.Cu") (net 25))
 (segment (start 60.96 76.591701) (end 55.001701 82.55) (width 0.25) (layer "B.Cu") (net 25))
 (segment (start 55.001701 82.55) (end 41.91 82.55) (width 0.25) (layer "B.Cu") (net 25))
 (segment (start 66.97 58.69) (end 77.74 58.69) (width 0.25) (layer "F.Cu") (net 29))
 (segment (start 77.74 58.69) (end 82.55 63.5) (width 0.25) (layer "F.Cu") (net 29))
 (segment (start 81.995 65.325) (end 82.55 65.325) (width 0.25) (layer "F.Cu") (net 31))
 (segment (start 58.42 88.9) (end 81.995 65.325) (width 0.25) (layer "F.Cu") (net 31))
 (segment (start 52.07 88.9) (end 58.42 88.9) (width 0.25) (layer "F.Cu") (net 31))
 (segment (start 74.43 59.19) (end 78.74 63.5) (width 0.25) (layer "F.Cu") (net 16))
 (segment (start 66.97 59.19) (end 74.43 59.19) (width 0.25) (layer "F.Cu") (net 16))
 (segment (start 78.74 66.04) (end 58.42 86.36) (width 0.25) (layer "F.Cu") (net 17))
 (segment (start 58.42 86.36) (end 52.07 86.36) (width 0.25) (layer "F.Cu") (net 17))
 (segment (start 52.07 86.36) (end 49.53 88.9) (width 0.25) (layer "F.Cu") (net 17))
 (segment (start 78.74 65.325) (end 78.74 66.04) (width 0.25) (layer "F.Cu") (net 17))
 (segment (start 66.97 59.69) (end 71.12 59.69) (width 0.25) (layer "F.Cu") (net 28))
 (segment (start 71.12 59.69) (end 74.93 63.5) (width 0.25) (layer "F.Cu") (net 28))
 (segment (start 57.15 85.09) (end 50.8 85.09) (width 0.25) (layer "F.Cu") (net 33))
 (segment (start 50.8 85.09) (end 46.99 88.9) (width 0.25) (layer "F.Cu") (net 33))
 (segment (start 74.93 67.31) (end 57.15 85.09) (width 0.25) (layer "F.Cu") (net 33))
 (segment (start 74.93 65.325) (end 74.93 67.31) (width 0.25) (layer "F.Cu") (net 33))
 (segment (start 67.81 60.19) (end 71.12 63.5) (width 0.25) (layer "F.Cu") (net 27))
 (segment (start 66.97 60.19) (end 67.81 60.19) (width 0.25) (layer "F.Cu") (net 27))
 (segment (start 71.12 68.483375) (end 55.783375 83.82) (width 0.25) (layer "F.Cu") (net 30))
 (segment (start 71.12 65.325) (end 71.12 68.483375) (width 0.25) (layer "F.Cu") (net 30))
 (segment (start 55.783375 83.82) (end 49.53 83.82) (width 0.25) (layer "F.Cu") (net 30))
 (segment (start 49.53 83.82) (end 44.45 88.9) (width 0.25) (layer "F.Cu") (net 30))
 (segment (start 66.97 60.69) (end 66.97 63.16) (width 0.25) (layer "F.Cu") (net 26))
 (segment (start 66.97 63.16) (end 67.31 63.5) (width 0.25) (layer "F.Cu") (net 26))
 (segment (start 39.37 84.7325) (end 39.37 88.9) (width 0.25) (layer "F.Cu") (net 32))
 (segment (start 36.83 43.18) (end 39.37 43.18) (width 0.25) (layer "F.Cu") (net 34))
 (segment (start 39.37 45.72) (end 36.83 45.72) (width 0.25) (layer "F.Cu") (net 35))
 (segment (start 36.83 48.26) (end 39.37 48.26) (width 0.25) (layer "F.Cu") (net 36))
 (segment (start 39.37 50.8) (end 36.83 50.8) (width 0.25) (layer "F.Cu") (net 37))
 (segment (start 36.83 53.34) (end 39.37 53.34) (width 0.25) (layer "F.Cu") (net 38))
 (segment (start 39.37 55.88) (end 36.83 55.88) (width 0.25) (layer "F.Cu") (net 39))
 (segment (start 36.83 58.42) (end 39.37 58.42) (width 0.25) (layer "F.Cu") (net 40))
 (segment (start 36.83 60.96) (end 39.37 60.96) (width 0.25) (layer "F.Cu") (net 41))
 (segment (start 39.37 63.5) (end 36.83 63.5) (width 0.25) (layer "F.Cu") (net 42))
 (segment (start 36.83 66.04) (end 39.37 66.04) (width 0.25) (layer "F.Cu") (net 43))
 (segment (start 39.37 68.58) (end 36.83 68.58) (width 0.25) (layer "F.Cu") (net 44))
 (segment (start 39.37 73.66) (end 36.83 73.66) (width 0.25) (layer "F.Cu") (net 45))
 (segment (start 36.83 76.2) (end 39.37 76.2) (width 0.25) (layer "F.Cu") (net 46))
 (segment (start 39.37 78.74) (end 36.83 78.74) (width 0.25) (layer "F.Cu") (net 47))
 (segment (start 54.61 43.18) (end 57.15 43.18) (width 0.25) (layer "F.Cu") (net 1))
 (segment (start 57.15 45.72) (end 54.61 45.72) (width 0.25) (layer "F.Cu") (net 2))
 (segment (start 54.61 48.26) (end 57.15 48.26) (width 0.25) (layer "F.Cu") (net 3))
 (segment (start 57.15 50.8) (end 54.61 50.8) (width 0.25) (layer "F.Cu") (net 4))
 (segment (start 54.61 53.34) (end 57.15 53.34) (width 0.25) (layer "F.Cu") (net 5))
 (segment (start 57.15 55.88) (end 54.61 55.88) (width 0.25) (layer "F.Cu") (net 6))
 (segment (start 54.61 58.42) (end 57.15 58.42) (width 0.25) (layer "F.Cu") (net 7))
 (segment (start 54.61 60.96) (end 57.15 60.96) (width 0.25) (layer "F.Cu") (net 8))
 (segment (start 57.15 63.5) (end 54.61 63.5) (width 0.25) (layer "F.Cu") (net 9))
 (segment (start 54.61 66.04) (end 57.15 66.04) (width 0.25) (layer "F.Cu") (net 10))
 (segment (start 57.15 68.58) (end 54.61 68.58) (width 0.25) (layer "F.Cu") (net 11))
 (segment (start 54.61 68.58) (end 52.07 68.58) (width 0.25) (layer "F.Cu") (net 11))
 (segment (start 57.9875 69.4175) (end 57.15 68.58) (width 0.25) (layer "F.Cu") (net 11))
 (segment (start 67.31 65.325) (end 65.82 66.815) (width 0.25) (layer "F.Cu") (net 11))
 (segment (start 65.82 69.068173) (end 65.470673 69.4175) (width 0.25) (layer "F.Cu") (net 11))
 (segment (start 41.91 88.9) (end 50.287348 80.522652) (width 0.25) (layer "F.Cu") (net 11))
 (segment (start 65.470673 69.4175) (end 57.9875 69.4175) (width 0.25) (layer "F.Cu") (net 11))
 (segment (start 65.82 66.815) (end 65.82 69.068173) (width 0.25) (layer "F.Cu") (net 11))
 (segment (start 50.287348 80.522652) (end 50.287348 74.172652) (width 0.25) (layer "F.Cu") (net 11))
 (via (at 52.07 68.58) (size 0.8) (drill 0.4) (layers "F.Cu" "B.Cu") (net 11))
 (via (at 50.287348 74.172652) (size 0.8) (drill 0.4) (layers "F.Cu" "B.Cu") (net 11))
 (segment (start 50.287348 74.172652) (end 50.287348 70.362652) (width 0.25) (layer "B.Cu") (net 11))
 (segment (start 50.287348 70.362652) (end 52.07 68.58) (width 0.25) (layer "B.Cu") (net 11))
 (segment (start 57.15 73.66) (end 54.61 73.66) (width 0.25) (layer "F.Cu") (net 13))
 (segment (start 54.61 76.2) (end 57.15 76.2) (width 0.25) (layer "F.Cu") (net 14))
 (segment (start 57.15 78.74) (end 54.61 78.74) (width 0.25) (layer "F.Cu") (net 15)))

